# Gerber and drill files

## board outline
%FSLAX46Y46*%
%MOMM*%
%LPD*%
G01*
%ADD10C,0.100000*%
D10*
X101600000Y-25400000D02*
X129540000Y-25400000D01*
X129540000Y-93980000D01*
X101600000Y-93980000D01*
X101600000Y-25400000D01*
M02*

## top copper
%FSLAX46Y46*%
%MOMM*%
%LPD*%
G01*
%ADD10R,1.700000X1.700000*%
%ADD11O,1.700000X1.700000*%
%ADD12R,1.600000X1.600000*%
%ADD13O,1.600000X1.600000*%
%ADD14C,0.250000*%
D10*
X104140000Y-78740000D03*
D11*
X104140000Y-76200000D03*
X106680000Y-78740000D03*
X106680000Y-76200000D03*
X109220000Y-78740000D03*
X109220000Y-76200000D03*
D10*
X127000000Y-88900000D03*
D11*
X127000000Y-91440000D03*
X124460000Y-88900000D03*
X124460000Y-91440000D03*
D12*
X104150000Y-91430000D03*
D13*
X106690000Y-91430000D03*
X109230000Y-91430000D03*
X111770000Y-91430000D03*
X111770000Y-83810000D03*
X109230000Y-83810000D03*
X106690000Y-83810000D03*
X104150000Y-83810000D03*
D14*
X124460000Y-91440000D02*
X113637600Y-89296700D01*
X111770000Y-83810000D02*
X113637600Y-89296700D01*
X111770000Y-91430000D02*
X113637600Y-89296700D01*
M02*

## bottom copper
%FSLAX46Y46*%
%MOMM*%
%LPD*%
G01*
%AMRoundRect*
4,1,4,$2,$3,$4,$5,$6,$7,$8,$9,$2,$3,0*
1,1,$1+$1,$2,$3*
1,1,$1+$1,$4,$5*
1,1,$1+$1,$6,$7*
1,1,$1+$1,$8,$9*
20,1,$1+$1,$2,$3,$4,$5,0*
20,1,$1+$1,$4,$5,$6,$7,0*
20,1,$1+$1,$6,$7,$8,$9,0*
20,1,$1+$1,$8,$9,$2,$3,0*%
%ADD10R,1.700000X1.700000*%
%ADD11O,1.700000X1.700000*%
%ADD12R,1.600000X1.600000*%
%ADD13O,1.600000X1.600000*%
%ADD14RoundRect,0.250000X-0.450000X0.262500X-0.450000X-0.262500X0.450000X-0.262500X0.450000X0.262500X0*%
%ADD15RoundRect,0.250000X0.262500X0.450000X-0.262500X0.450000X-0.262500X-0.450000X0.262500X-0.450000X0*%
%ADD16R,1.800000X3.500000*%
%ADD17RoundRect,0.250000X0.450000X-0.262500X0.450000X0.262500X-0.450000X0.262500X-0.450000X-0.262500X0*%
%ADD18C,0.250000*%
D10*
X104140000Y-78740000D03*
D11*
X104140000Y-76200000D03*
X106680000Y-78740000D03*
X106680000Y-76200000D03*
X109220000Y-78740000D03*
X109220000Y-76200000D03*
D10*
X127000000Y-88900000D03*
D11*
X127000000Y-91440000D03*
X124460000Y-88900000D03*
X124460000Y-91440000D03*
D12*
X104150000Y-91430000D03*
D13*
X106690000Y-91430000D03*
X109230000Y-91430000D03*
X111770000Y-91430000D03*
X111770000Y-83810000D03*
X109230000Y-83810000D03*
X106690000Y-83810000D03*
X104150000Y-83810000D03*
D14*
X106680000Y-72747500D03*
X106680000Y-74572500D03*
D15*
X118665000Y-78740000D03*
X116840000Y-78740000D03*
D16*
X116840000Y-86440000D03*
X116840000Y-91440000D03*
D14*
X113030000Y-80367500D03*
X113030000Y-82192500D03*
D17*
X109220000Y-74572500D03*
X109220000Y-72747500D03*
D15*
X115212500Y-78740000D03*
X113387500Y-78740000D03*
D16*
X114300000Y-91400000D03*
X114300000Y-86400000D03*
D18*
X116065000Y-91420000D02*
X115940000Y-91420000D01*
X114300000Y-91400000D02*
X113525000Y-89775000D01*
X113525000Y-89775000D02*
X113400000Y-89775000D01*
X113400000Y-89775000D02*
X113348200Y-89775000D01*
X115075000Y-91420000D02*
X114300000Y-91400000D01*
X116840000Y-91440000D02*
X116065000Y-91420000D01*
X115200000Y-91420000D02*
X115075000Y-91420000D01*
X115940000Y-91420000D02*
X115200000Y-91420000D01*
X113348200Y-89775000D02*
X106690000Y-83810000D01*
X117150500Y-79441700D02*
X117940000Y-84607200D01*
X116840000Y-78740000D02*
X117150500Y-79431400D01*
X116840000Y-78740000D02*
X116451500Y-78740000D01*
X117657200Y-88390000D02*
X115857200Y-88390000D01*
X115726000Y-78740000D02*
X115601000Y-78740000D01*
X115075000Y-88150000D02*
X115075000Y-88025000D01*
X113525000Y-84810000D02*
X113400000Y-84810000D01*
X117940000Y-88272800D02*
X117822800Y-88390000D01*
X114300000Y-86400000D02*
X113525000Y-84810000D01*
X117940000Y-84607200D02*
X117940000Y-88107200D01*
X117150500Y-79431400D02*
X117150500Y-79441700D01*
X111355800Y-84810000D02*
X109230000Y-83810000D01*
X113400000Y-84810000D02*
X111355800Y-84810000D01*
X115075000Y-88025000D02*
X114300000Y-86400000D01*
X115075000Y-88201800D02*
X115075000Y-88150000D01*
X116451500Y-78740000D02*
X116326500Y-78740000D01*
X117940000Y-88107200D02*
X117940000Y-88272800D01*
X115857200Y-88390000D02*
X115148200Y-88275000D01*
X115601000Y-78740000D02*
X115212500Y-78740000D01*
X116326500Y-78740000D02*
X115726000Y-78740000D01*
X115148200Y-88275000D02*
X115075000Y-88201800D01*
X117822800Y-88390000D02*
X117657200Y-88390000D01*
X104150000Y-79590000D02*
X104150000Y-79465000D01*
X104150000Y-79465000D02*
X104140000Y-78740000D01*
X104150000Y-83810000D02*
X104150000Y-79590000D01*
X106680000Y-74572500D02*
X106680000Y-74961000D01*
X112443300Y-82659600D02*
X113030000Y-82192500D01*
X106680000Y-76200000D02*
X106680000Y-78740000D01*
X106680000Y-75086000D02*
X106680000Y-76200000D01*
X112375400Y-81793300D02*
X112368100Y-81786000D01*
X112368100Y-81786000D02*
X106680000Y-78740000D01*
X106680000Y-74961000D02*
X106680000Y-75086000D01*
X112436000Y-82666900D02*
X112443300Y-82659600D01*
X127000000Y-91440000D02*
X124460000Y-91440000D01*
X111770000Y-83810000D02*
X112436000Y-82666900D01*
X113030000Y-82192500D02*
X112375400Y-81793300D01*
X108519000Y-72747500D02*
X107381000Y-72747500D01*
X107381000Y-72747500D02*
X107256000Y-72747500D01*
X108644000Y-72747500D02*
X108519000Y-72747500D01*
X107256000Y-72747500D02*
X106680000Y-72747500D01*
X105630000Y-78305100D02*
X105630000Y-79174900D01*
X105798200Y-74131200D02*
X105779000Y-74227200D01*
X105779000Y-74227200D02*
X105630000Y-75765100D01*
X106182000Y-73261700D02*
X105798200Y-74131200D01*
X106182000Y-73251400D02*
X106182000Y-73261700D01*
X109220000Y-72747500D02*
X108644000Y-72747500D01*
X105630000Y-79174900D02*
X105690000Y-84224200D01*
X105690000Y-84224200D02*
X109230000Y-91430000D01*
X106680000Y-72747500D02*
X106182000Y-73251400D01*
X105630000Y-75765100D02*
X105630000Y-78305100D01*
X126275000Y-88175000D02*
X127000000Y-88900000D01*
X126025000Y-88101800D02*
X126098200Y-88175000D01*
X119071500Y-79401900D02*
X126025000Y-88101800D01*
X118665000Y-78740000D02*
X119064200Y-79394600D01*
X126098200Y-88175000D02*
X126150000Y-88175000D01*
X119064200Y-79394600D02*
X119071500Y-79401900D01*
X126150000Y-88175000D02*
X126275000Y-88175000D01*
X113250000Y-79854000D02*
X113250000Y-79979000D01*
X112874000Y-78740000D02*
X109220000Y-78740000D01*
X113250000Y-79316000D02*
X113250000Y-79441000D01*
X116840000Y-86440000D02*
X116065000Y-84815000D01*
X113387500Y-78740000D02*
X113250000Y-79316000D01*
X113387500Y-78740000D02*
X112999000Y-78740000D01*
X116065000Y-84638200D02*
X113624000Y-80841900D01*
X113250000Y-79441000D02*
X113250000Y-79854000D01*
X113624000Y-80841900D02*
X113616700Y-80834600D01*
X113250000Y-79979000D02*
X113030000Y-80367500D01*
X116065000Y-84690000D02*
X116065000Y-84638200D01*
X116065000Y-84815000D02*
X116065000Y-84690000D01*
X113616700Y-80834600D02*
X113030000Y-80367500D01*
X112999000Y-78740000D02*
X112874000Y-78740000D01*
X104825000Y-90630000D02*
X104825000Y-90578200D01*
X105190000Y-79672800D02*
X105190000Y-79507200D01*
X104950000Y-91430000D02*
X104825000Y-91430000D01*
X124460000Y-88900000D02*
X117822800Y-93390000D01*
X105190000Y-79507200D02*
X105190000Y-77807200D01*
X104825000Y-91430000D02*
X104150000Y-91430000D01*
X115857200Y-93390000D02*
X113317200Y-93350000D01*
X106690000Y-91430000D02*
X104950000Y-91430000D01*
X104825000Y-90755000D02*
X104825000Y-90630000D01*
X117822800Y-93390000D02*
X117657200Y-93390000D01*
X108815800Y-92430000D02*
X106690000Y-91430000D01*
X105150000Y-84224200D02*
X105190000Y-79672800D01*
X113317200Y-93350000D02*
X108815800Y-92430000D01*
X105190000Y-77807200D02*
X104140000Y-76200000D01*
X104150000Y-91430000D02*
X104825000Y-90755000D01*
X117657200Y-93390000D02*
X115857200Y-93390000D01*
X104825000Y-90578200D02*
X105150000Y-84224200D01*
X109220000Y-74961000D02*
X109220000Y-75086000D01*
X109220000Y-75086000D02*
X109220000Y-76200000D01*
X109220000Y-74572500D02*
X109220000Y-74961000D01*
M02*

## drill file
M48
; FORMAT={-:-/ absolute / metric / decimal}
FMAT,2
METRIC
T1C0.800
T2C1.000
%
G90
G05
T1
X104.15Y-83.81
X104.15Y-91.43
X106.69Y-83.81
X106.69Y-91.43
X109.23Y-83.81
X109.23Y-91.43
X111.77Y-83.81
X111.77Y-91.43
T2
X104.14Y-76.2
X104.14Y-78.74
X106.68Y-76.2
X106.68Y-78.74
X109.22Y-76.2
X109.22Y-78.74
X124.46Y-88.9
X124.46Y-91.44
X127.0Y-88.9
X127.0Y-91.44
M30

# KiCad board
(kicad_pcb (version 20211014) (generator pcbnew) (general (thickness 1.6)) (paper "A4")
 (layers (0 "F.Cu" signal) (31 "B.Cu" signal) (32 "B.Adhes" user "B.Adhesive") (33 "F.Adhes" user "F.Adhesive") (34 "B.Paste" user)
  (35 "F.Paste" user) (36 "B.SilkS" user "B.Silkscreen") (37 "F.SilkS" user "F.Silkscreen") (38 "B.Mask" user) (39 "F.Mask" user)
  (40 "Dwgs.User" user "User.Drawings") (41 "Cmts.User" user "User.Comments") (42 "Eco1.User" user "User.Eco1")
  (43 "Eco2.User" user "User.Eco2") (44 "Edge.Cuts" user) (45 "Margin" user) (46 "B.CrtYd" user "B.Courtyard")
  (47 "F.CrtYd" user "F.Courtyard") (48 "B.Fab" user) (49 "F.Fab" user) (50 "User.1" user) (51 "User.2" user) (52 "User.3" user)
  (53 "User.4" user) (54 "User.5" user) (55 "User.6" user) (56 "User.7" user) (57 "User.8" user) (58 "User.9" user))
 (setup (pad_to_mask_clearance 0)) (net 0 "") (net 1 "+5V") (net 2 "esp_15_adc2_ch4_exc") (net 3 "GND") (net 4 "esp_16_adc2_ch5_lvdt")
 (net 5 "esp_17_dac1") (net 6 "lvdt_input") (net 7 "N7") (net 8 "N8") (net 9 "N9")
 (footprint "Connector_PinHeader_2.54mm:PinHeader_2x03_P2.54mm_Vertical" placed (layer "F.Cu") (at 104.14 78.74 90)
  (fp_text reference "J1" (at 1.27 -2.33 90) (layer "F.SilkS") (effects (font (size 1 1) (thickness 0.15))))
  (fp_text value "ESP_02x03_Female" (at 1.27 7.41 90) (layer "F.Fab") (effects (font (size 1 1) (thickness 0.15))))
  (pad "1" thru_hole rect (at 0 0 90) (size 1.7 1.7) (drill 1) (layers *.Cu *.Mask) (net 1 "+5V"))
  (pad "2" thru_hole oval (at 2.54 0 90) (size 1.7 1.7) (drill 1) (layers *.Cu *.Mask) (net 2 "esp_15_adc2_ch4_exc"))
  (pad "3" thru_hole oval (at 0 2.54 90) (size 1.7 1.7) (drill 1) (layers *.Cu *.Mask) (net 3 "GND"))
  (pad "4" thru_hole oval (at 2.54 2.54 90) (size 1.7 1.7) (drill 1) (layers *.Cu *.Mask) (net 3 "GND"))
  (pad "5" thru_hole oval (at 0 5.08 90) (size 1.7 1.7) (drill 1) (layers *.Cu *.Mask) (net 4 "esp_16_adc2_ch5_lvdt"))
  (pad "6" thru_hole oval (at 2.54 5.08 90) (size 1.7 1.7) (drill 1) (layers *.Cu *.Mask) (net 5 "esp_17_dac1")))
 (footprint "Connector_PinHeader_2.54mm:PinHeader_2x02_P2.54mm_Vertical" (layer "F.Cu") (at 127 88.9 -90)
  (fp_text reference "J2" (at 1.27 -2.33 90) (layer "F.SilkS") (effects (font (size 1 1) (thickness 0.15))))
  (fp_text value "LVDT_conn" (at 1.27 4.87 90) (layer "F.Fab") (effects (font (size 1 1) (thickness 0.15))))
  (pad "1" thru_hole rect (at 0 0 270) (size 1.7 1.7) (drill 1) (layers *.Cu *.Mask) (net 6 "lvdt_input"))
  (pad "2" thru_hole oval (at 2.54 0 270) (size 1.7 1.7) (drill 1) (layers *.Cu *.Mask) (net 3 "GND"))
  (pad "3" thru_hole oval (at 0 2.54 270) (size 1.7 1.7) (drill 1) (layers *.Cu *.Mask) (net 2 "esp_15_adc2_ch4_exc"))
  (pad "4" thru_hole oval (at 2.54 2.54 270) (size 1.7 1.7) (drill 1) (layers *.Cu *.Mask) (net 3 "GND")))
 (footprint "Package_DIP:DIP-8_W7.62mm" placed (layer "F.Cu") (at 104.15 91.43 90)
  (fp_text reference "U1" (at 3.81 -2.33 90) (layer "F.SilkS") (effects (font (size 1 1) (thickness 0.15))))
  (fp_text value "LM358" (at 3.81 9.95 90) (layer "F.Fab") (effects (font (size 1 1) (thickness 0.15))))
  (pad "1" thru_hole rect (at 0 0 90) (size 1.6 1.6) (drill 0.8) (layers *.Cu *.Mask) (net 2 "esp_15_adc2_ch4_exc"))
  (pad "2" thru_hole oval (at 0 2.54 90) (size 1.6 1.6) (drill 0.8) (layers *.Cu *.Mask) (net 2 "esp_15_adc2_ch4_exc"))
  (pad "3" thru_hole oval (at 0 5.08 90) (size 1.6 1.6) (drill 0.8) (layers *.Cu *.Mask) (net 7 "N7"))
  (pad "4" thru_hole oval (at 0 7.62 90) (size 1.6 1.6) (drill 0.8) (layers *.Cu *.Mask) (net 3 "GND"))
  (pad "5" thru_hole oval (at 7.62 7.62 90) (size 1.6 1.6) (drill 0.8) (layers *.Cu *.Mask) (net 3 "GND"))
  (pad "6" thru_hole oval (at 7.62 5.08 90) (size 1.6 1.6) (drill 0.8) (layers *.Cu *.Mask) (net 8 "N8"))
  (pad "7" thru_hole oval (at 7.62 2.54 90) (size 1.6 1.6) (drill 0.8) (layers *.Cu *.Mask) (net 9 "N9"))
  (pad "8" thru_hole oval (at 7.62 0 90) (size 1.6 1.6) (drill 0.8) (layers *.Cu *.Mask) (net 1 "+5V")))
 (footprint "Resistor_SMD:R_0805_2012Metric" (layer "B.Cu") (at 106.68 73.66 -90)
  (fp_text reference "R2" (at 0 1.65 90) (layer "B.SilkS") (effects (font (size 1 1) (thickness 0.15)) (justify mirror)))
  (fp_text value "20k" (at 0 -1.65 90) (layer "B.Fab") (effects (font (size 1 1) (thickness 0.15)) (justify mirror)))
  (pad "1" smd roundrect (at -0.9125 0 270) (size 1.025 1.4) (layers "B.Cu" "B.Paste" "B.Mask") (roundrect_rratio 0.243902) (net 7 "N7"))
  (pad "2" smd roundrect (at 0.9125 0 270) (size 1.025 1.4) (layers "B.Cu" "B.Paste" "B.Mask") (roundrect_rratio 0.243902) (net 3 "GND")))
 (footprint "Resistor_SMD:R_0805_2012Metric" (layer "B.Cu") (at 117.7525 78.74 180)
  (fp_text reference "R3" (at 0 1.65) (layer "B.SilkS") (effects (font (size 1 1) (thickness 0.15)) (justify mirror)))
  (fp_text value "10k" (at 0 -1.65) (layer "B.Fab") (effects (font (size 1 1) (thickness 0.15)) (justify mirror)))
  (pad "1" smd roundrect (at -0.9125 0 180) (size 1.025 1.4) (layers "B.Cu" "B.Paste" "B.Mask") (roundrect_rratio 0.243902)
   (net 6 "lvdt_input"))
  (pad "2" smd roundrect (at 0.9125 0 180) (size 1.025 1.4) (layers "B.Cu" "B.Paste" "B.Mask") (roundrect_rratio 0.243902) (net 8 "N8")))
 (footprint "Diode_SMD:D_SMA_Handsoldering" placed (layer "B.Cu") (at 116.84 88.94 -90)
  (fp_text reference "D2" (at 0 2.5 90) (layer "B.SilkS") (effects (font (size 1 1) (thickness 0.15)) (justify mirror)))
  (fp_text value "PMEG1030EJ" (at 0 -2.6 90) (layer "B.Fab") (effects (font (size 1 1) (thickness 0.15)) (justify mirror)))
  (pad "1" smd rect (at -2.5 0 270) (size 3.5 1.8) (layers "B.Cu" "B.Paste" "B.Mask") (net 4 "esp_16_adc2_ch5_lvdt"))
  (pad "2" smd rect (at 2.5 0 270) (size 3.5 1.8) (layers "B.Cu" "B.Paste" "B.Mask") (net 9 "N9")))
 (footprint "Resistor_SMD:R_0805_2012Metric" (layer "B.Cu") (at 113.03 81.28 -90)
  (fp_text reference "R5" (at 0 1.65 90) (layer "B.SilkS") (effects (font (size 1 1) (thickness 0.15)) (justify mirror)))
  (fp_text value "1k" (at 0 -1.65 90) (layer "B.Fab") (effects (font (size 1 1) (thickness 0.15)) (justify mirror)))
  (pad "1" smd roundrect (at -0.9125 0 270) (size 1.025 1.4) (layers "B.Cu" "B.Paste" "B.Mask") (roundrect_rratio 0.243902)
   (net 4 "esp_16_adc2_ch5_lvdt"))
  (pad "2" smd roundrect (at 0.9125 0 270) (size 1.025 1.4) (layers "B.Cu" "B.Paste" "B.Mask") (roundrect_rratio 0.243902) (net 3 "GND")))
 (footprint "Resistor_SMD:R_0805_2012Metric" (layer "B.Cu") (at 109.22 73.66 90)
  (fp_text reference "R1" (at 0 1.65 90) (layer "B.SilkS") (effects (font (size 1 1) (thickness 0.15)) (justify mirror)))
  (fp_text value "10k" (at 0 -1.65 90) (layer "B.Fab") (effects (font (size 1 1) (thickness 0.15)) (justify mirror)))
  (pad "1" smd roundrect (at -0.9125 0 90) (size 1.025 1.4) (layers "B.Cu" "B.Paste" "B.Mask") (roundrect_rratio 0.243902)
   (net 5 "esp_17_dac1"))
  (pad "2" smd roundrect (at 0.9125 0 90) (size 1.025 1.4) (layers "B.Cu" "B.Paste" "B.Mask") (roundrect_rratio 0.243902) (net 7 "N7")))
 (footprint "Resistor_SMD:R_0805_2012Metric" (layer "B.Cu") (at 114.3 78.74 180)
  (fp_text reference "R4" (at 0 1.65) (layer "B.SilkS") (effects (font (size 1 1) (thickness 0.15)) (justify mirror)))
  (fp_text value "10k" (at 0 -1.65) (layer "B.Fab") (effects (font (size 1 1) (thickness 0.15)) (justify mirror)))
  (pad "1" smd roundrect (at -0.9125 0 180) (size 1.025 1.4) (layers "B.Cu" "B.Paste" "B.Mask") (roundrect_rratio 0.243902) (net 8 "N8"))
  (pad "2" smd roundrect (at 0.9125 0 180) (size 1.025 1.4) (layers "B.Cu" "B.Paste" "B.Mask") (roundrect_rratio 0.243902)
   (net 4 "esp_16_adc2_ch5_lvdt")))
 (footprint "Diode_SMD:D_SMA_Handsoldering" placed (layer "B.Cu") (at 114.3 88.9 90)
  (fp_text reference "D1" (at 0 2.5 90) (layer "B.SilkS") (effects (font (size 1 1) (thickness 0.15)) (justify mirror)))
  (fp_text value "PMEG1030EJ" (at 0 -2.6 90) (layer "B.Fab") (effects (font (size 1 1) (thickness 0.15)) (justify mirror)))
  (pad "1" smd rect (at -2.5 0 90) (size 3.5 1.8) (layers "B.Cu" "B.Paste" "B.Mask") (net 9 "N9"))
  (pad "2" smd rect (at 2.5 0 90) (size 3.5 1.8) (layers "B.Cu" "B.Paste" "B.Mask") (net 8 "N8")))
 (gr_rect (start 101.6 25.4) (end 129.54 93.98) (layer "Edge.Cuts") (width 0.1) (fill none))
 (segment (start 116.065 91.42) (end 115.94 91.42) (width 0.25) (layer "B.Cu") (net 9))
 (segment (start 114.3 91.4) (end 113.525 89.775) (width 0.25) (layer "B.Cu") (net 9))
 (segment (start 113.525 89.775) (end 113.4 89.775) (width 0.25) (layer "B.Cu") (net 9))
 (segment (start 113.4 89.775) (end 113.3482 89.775) (width 0.25) (layer "B.Cu") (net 9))
 (segment (start 115.075 91.42) (end 114.3 91.4) (width 0.25) (layer "B.Cu") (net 9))
 (segment (start 116.84 91.44) (end 116.065 91.42) (width 0.25) (layer "B.Cu") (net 9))
 (segment (start 115.2 91.42) (end 115.075 91.42) (width 0.25) (layer "B.Cu") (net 9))
 (segment (start 115.94 91.42) (end 115.2 91.42) (width 0.25) (layer "B.Cu") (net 9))
 (segment (start 113.3482 89.775) (end 106.69 83.81) (width 0.25) (layer "B.Cu") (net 9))
 (segment (start 117.1505 79.4417) (end 117.94 84.6072) (width 0.25) (layer "B.Cu") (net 8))
 (segment (start 116.84 78.74) (end 117.1505 79.4314) (width 0.25) (layer "B.Cu") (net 8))
 (segment (start 116.84 78.74) (end 116.4515 78.74) (width 0.25) (layer "B.Cu") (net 8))
 (segment (start 117.6572 88.39) (end 115.8572 88.39) (width 0.25) (layer "B.Cu") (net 8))
 (segment (start 115.726 78.74) (end 115.601 78.74) (width 0.25) (layer "B.Cu") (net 8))
 (segment (start 115.075 88.15) (end 115.075 88.025) (width 0.25) (layer "B.Cu") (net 8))
 (segment (start 113.525 84.81) (end 113.4 84.81) (width 0.25) (layer "B.Cu") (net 8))
 (segment (start 117.94 88.2728) (end 117.8228 88.39) (width 0.25) (layer "B.Cu") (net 8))
 (segment (start 114.3 86.4) (end 113.525 84.81) (width 0.25) (layer "B.Cu") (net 8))
 (segment (start 117.94 84.6072) (end 117.94 88.1072) (width 0.25) (layer "B.Cu") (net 8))
 (segment (start 117.1505 79.4314) (end 117.1505 79.4417) (width 0.25) (layer "B.Cu") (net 8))
 (segment (start 111.3558 84.81) (end 109.23 83.81) (width 0.25) (layer "B.Cu") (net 8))
 (segment (start 113.4 84.81) (end 111.3558 84.81) (width 0.25) (layer "B.Cu") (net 8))
 (segment (start 115.075 88.025) (end 114.3 86.4) (width 0.25) (layer "B.Cu") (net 8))
 (segment (start 115.075 88.2018) (end 115.075 88.15) (width 0.25) (layer "B.Cu") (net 8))
 (segment (start 116.4515 78.74) (end 116.3265 78.74) (width 0.25) (layer "B.Cu") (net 8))
 (segment (start 117.94 88.1072) (end 117.94 88.2728) (width 0.25) (layer "B.Cu") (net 8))
 (segment (start 115.8572 88.39) (end 115.1482 88.275) (width 0.25) (layer "B.Cu") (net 8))
 (segment (start 115.601 78.74) (end 115.2125 78.74) (width 0.25) (layer "B.Cu") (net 8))
 (segment (start 116.3265 78.74) (end 115.726 78.74) (width 0.25) (layer "B.Cu") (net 8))
 (segment (start 115.1482 88.275) (end 115.075 88.2018) (width 0.25) (layer "B.Cu") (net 8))
 (segment (start 117.8228 88.39) (end 117.6572 88.39) (width 0.25) (layer "B.Cu") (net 8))
 (segment (start 104.15 79.59) (end 104.15 79.465) (width 0.25) (layer "B.Cu") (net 1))
 (segment (start 104.15 79.465) (end 104.14 78.74) (width 0.25) (layer "B.Cu") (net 1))
 (segment (start 104.15 83.81) (end 104.15 79.59) (width 0.25) (layer "B.Cu") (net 1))
 (segment (start 124.46 91.44) (end 113.6376 89.2967) (width 0.25) (layer "F.Cu") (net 3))
 (segment (start 111.77 83.81) (end 113.6376 89.2967) (width 0.25) (layer "F.Cu") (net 3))
 (segment (start 111.77 91.43) (end 113.6376 89.2967) (width 0.25) (layer "F.Cu") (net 3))
 (segment (start 106.68 74.5725) (end 106.68 74.961) (width 0.25) (layer "B.Cu") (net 3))
 (segment (start 112.4433 82.6596) (end 113.03 82.1925) (width 0.25) (layer "B.Cu") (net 3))
 (segment (start 106.68 76.2) (end 106.68 78.74) (width 0.25) (layer "B.Cu") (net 3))
 (segment (start 106.68 75.086) (end 106.68 76.2) (width 0.25) (layer "B.Cu") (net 3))
 (segment (start 112.3754 81.7933) (end 112.3681 81.786) (width 0.25) (layer "B.Cu") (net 3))
 (segment (start 112.3681 81.786) (end 106.68 78.74) (width 0.25) (layer "B.Cu") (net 3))
 (segment (start 106.68 74.961) (end 106.68 75.086) (width 0.25) (layer "B.Cu") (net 3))
 (segment (start 112.436 82.6669) (end 112.4433 82.6596) (width 0.25) (layer "B.Cu") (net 3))
 (segment (start 127 91.44) (end 124.46 91.44) (width 0.25) (layer "B.Cu") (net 3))
 (segment (start 111.77 83.81) (end 112.436 82.6669) (width 0.25) (layer "B.Cu") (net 3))
 (segment (start 113.03 82.1925) (end 112.3754 81.7933) (width 0.25) (layer "B.Cu") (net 3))
 (segment (start 108.519 72.7475) (end 107.381 72.7475) (width 0.25) (layer "B.Cu") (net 7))
 (segment (start 107.381 72.7475) (end 107.256 72.7475) (width 0.25) (layer "B.Cu") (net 7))
 (segment (start 108.644 72.7475) (end 108.519 72.7475) (width 0.25) (layer "B.Cu") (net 7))
 (segment (start 107.256 72.7475) (end 106.68 72.7475) (width 0.25) (layer "B.Cu") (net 7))
 (segment (start 105.63 78.3051) (end 105.63 79.1749) (width 0.25) (layer "B.Cu") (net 7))
 (segment (start 105.7982 74.1312) (end 105.779 74.2272) (width 0.25) (layer "B.Cu") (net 7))
 (segment (start 105.779 74.2272) (end 105.63 75.7651) (width 0.25) (layer "B.Cu") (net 7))
 (segment (start 106.182 73.2617) (end 105.7982 74.1312) (width 0.25) (layer "B.Cu") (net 7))
 (segment (start 106.182 73.2514) (end 106.182 73.2617) (width 0.25) (layer "B.Cu") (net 7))
 (segment (start 109.22 72.7475) (end 108.644 72.7475) (width 0.25) (layer "B.Cu") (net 7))
 (segment (start 105.63 79.1749) (end 105.69 84.2242) (width 0.25) (layer "B.Cu") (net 7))
 (segment (start 105.69 84.2242) (end 109.23 91.43) (width 0.25) (layer "B.Cu") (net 7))
 (segment (start 106.68 72.7475) (end 106.182 73.2514) (width 0.25) (layer "B.Cu") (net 7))
 (segment (start 105.63 75.7651) (end 105.63 78.3051) (width 0.25) (layer "B.Cu") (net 7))
 (segment (start 126.275 88.175) (end 127 88.9) (width 0.25) (layer "B.Cu") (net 6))
 (segment (start 126.025 88.1018) (end 126.0982 88.175) (width 0.25) (layer "B.Cu") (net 6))
 (segment (start 119.0715 79.4019) (end 126.025 88.1018) (width 0.25) (layer "B.Cu") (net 6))
 (segment (start 118.665 78.74) (end 119.0642 79.3946) (width 0.25) (layer "B.Cu") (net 6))
 (segment (start 126.0982 88.175) (end 126.15 88.175) (width 0.25) (layer "B.Cu") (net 6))
 (segment (start 119.0642 79.3946) (end 119.0715 79.4019) (width 0.25) (layer "B.Cu") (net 6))
 (segment (start 126.15 88.175) (end 126.275 88.175) (width 0.25) (layer "B.Cu") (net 6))
 (segment (start 113.25 79.854) (end 113.25 79.979) (width 0.25) (layer "B.Cu") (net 4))
 (segment (start 112.874 78.74) (end 109.22 78.74) (width 0.25) (layer "B.Cu") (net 4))
 (segment (start 113.25 79.316) (end 113.25 79.441) (width 0.25) (layer "B.Cu") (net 4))
 (segment (start 116.84 86.44) (end 116.065 84.815) (width 0.25) (layer "B.Cu") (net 4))
 (segment (start 113.3875 78.74) (end 113.25 79.316) (width 0.25) (layer "B.Cu") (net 4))
 (segment (start 113.3875 78.74) (end 112.999 78.74) (width 0.25) (layer "B.Cu") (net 4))
 (segment (start 116.065 84.6382) (end 113.624 80.8419) (width 0.25) (layer "B.Cu") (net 4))
 (segment (start 113.25 79.441) (end 113.25 79.854) (width 0.25) (layer "B.Cu") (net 4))
 (segment (start 113.624 80.8419) (end 113.6167 80.8346) (width 0.25) (layer "B.Cu") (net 4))
 (segment (start 113.25 79.979) (end 113.03 80.3675) (width 0.25) (layer "B.Cu") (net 4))
 (segment (start 116.065 84.69) (end 116.065 84.6382) (width 0.25) (layer "B.Cu") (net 4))
 (segment (start 116.065 84.815) (end 116.065 84.69) (width 0.25) (layer "B.Cu") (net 4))
 (segment (start 113.6167 80.8346) (end 113.03 80.3675) (width 0.25) (layer "B.Cu") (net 4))
 (segment (start 112.999 78.74) (end 112.874 78.74) (width 0.25) (layer "B.Cu") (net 4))
 (segment (start 104.825 90.63) (end 104.825 90.5782) (width 0.25) (layer "B.Cu") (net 2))
 (segment (start 105.19 79.6728) (end 105.19 79.5072) (width 0.25) (layer "B.Cu") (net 2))
 (segment (start 104.95 91.43) (end 104.825 91.43) (width 0.25) (layer "B.Cu") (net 2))
 (segment (start 124.46 88.9) (end 117.8228 93.39) (width 0.25) (layer "B.Cu") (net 2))
 (segment (start 105.19 79.5072) (end 105.19 77.8072) (width 0.25) (layer "B.Cu") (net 2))
 (segment (start 104.825 91.43) (end 104.15 91.43) (width 0.25) (layer "B.Cu") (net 2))
 (segment (start 115.8572 93.39) (end 113.3172 93.35) (width 0.25) (layer "B.Cu") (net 2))
 (segment (start 106.69 91.43) (end 104.95 91.43) (width 0.25) (layer "B.Cu") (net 2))
 (segment (start 104.825 90.755) (end 104.825 90.63) (width 0.25) (layer "B.Cu") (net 2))
 (segment (start 117.8228 93.39) (end 117.6572 93.39) (width 0.25) (layer "B.Cu") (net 2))
 (segment (start 108.8158 92.43) (end 106.69 91.43) (width 0.25) (layer "B.Cu") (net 2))
 (segment (start 105.15 84.2242) (end 105.19 79.6728) (width 0.25) (layer "B.Cu") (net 2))
 (segment (start 113.3172 93.35) (end 108.8158 92.43) (width 0.25) (layer "B.Cu") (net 2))
 (segment (start 105.19 77.8072) (end 104.14 76.2) (width 0.25) (layer "B.Cu") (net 2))
 (segment (start 104.15 91.43) (end 104.825 90.755) (width 0.25) (layer "B.Cu") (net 2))
 (segment (start 117.6572 93.39) (end 115.8572 93.39) (width 0.25) (layer "B.Cu") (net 2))
 (segment (start 104.825 90.5782) (end 105.15 84.2242) (width 0.25) (layer "B.Cu") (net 2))
 (segment (start 109.22 74.961) (end 109.22 75.086) (width 0.25) (layer "B.Cu") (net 5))
 (segment (start 109.22 75.086) (end 109.22 76.2) (width 0.25) (layer "B.Cu") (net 5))
 (segment (start 109.22 74.5725) (end 109.22 74.961) (width 0.25) (layer "B.Cu") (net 5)))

